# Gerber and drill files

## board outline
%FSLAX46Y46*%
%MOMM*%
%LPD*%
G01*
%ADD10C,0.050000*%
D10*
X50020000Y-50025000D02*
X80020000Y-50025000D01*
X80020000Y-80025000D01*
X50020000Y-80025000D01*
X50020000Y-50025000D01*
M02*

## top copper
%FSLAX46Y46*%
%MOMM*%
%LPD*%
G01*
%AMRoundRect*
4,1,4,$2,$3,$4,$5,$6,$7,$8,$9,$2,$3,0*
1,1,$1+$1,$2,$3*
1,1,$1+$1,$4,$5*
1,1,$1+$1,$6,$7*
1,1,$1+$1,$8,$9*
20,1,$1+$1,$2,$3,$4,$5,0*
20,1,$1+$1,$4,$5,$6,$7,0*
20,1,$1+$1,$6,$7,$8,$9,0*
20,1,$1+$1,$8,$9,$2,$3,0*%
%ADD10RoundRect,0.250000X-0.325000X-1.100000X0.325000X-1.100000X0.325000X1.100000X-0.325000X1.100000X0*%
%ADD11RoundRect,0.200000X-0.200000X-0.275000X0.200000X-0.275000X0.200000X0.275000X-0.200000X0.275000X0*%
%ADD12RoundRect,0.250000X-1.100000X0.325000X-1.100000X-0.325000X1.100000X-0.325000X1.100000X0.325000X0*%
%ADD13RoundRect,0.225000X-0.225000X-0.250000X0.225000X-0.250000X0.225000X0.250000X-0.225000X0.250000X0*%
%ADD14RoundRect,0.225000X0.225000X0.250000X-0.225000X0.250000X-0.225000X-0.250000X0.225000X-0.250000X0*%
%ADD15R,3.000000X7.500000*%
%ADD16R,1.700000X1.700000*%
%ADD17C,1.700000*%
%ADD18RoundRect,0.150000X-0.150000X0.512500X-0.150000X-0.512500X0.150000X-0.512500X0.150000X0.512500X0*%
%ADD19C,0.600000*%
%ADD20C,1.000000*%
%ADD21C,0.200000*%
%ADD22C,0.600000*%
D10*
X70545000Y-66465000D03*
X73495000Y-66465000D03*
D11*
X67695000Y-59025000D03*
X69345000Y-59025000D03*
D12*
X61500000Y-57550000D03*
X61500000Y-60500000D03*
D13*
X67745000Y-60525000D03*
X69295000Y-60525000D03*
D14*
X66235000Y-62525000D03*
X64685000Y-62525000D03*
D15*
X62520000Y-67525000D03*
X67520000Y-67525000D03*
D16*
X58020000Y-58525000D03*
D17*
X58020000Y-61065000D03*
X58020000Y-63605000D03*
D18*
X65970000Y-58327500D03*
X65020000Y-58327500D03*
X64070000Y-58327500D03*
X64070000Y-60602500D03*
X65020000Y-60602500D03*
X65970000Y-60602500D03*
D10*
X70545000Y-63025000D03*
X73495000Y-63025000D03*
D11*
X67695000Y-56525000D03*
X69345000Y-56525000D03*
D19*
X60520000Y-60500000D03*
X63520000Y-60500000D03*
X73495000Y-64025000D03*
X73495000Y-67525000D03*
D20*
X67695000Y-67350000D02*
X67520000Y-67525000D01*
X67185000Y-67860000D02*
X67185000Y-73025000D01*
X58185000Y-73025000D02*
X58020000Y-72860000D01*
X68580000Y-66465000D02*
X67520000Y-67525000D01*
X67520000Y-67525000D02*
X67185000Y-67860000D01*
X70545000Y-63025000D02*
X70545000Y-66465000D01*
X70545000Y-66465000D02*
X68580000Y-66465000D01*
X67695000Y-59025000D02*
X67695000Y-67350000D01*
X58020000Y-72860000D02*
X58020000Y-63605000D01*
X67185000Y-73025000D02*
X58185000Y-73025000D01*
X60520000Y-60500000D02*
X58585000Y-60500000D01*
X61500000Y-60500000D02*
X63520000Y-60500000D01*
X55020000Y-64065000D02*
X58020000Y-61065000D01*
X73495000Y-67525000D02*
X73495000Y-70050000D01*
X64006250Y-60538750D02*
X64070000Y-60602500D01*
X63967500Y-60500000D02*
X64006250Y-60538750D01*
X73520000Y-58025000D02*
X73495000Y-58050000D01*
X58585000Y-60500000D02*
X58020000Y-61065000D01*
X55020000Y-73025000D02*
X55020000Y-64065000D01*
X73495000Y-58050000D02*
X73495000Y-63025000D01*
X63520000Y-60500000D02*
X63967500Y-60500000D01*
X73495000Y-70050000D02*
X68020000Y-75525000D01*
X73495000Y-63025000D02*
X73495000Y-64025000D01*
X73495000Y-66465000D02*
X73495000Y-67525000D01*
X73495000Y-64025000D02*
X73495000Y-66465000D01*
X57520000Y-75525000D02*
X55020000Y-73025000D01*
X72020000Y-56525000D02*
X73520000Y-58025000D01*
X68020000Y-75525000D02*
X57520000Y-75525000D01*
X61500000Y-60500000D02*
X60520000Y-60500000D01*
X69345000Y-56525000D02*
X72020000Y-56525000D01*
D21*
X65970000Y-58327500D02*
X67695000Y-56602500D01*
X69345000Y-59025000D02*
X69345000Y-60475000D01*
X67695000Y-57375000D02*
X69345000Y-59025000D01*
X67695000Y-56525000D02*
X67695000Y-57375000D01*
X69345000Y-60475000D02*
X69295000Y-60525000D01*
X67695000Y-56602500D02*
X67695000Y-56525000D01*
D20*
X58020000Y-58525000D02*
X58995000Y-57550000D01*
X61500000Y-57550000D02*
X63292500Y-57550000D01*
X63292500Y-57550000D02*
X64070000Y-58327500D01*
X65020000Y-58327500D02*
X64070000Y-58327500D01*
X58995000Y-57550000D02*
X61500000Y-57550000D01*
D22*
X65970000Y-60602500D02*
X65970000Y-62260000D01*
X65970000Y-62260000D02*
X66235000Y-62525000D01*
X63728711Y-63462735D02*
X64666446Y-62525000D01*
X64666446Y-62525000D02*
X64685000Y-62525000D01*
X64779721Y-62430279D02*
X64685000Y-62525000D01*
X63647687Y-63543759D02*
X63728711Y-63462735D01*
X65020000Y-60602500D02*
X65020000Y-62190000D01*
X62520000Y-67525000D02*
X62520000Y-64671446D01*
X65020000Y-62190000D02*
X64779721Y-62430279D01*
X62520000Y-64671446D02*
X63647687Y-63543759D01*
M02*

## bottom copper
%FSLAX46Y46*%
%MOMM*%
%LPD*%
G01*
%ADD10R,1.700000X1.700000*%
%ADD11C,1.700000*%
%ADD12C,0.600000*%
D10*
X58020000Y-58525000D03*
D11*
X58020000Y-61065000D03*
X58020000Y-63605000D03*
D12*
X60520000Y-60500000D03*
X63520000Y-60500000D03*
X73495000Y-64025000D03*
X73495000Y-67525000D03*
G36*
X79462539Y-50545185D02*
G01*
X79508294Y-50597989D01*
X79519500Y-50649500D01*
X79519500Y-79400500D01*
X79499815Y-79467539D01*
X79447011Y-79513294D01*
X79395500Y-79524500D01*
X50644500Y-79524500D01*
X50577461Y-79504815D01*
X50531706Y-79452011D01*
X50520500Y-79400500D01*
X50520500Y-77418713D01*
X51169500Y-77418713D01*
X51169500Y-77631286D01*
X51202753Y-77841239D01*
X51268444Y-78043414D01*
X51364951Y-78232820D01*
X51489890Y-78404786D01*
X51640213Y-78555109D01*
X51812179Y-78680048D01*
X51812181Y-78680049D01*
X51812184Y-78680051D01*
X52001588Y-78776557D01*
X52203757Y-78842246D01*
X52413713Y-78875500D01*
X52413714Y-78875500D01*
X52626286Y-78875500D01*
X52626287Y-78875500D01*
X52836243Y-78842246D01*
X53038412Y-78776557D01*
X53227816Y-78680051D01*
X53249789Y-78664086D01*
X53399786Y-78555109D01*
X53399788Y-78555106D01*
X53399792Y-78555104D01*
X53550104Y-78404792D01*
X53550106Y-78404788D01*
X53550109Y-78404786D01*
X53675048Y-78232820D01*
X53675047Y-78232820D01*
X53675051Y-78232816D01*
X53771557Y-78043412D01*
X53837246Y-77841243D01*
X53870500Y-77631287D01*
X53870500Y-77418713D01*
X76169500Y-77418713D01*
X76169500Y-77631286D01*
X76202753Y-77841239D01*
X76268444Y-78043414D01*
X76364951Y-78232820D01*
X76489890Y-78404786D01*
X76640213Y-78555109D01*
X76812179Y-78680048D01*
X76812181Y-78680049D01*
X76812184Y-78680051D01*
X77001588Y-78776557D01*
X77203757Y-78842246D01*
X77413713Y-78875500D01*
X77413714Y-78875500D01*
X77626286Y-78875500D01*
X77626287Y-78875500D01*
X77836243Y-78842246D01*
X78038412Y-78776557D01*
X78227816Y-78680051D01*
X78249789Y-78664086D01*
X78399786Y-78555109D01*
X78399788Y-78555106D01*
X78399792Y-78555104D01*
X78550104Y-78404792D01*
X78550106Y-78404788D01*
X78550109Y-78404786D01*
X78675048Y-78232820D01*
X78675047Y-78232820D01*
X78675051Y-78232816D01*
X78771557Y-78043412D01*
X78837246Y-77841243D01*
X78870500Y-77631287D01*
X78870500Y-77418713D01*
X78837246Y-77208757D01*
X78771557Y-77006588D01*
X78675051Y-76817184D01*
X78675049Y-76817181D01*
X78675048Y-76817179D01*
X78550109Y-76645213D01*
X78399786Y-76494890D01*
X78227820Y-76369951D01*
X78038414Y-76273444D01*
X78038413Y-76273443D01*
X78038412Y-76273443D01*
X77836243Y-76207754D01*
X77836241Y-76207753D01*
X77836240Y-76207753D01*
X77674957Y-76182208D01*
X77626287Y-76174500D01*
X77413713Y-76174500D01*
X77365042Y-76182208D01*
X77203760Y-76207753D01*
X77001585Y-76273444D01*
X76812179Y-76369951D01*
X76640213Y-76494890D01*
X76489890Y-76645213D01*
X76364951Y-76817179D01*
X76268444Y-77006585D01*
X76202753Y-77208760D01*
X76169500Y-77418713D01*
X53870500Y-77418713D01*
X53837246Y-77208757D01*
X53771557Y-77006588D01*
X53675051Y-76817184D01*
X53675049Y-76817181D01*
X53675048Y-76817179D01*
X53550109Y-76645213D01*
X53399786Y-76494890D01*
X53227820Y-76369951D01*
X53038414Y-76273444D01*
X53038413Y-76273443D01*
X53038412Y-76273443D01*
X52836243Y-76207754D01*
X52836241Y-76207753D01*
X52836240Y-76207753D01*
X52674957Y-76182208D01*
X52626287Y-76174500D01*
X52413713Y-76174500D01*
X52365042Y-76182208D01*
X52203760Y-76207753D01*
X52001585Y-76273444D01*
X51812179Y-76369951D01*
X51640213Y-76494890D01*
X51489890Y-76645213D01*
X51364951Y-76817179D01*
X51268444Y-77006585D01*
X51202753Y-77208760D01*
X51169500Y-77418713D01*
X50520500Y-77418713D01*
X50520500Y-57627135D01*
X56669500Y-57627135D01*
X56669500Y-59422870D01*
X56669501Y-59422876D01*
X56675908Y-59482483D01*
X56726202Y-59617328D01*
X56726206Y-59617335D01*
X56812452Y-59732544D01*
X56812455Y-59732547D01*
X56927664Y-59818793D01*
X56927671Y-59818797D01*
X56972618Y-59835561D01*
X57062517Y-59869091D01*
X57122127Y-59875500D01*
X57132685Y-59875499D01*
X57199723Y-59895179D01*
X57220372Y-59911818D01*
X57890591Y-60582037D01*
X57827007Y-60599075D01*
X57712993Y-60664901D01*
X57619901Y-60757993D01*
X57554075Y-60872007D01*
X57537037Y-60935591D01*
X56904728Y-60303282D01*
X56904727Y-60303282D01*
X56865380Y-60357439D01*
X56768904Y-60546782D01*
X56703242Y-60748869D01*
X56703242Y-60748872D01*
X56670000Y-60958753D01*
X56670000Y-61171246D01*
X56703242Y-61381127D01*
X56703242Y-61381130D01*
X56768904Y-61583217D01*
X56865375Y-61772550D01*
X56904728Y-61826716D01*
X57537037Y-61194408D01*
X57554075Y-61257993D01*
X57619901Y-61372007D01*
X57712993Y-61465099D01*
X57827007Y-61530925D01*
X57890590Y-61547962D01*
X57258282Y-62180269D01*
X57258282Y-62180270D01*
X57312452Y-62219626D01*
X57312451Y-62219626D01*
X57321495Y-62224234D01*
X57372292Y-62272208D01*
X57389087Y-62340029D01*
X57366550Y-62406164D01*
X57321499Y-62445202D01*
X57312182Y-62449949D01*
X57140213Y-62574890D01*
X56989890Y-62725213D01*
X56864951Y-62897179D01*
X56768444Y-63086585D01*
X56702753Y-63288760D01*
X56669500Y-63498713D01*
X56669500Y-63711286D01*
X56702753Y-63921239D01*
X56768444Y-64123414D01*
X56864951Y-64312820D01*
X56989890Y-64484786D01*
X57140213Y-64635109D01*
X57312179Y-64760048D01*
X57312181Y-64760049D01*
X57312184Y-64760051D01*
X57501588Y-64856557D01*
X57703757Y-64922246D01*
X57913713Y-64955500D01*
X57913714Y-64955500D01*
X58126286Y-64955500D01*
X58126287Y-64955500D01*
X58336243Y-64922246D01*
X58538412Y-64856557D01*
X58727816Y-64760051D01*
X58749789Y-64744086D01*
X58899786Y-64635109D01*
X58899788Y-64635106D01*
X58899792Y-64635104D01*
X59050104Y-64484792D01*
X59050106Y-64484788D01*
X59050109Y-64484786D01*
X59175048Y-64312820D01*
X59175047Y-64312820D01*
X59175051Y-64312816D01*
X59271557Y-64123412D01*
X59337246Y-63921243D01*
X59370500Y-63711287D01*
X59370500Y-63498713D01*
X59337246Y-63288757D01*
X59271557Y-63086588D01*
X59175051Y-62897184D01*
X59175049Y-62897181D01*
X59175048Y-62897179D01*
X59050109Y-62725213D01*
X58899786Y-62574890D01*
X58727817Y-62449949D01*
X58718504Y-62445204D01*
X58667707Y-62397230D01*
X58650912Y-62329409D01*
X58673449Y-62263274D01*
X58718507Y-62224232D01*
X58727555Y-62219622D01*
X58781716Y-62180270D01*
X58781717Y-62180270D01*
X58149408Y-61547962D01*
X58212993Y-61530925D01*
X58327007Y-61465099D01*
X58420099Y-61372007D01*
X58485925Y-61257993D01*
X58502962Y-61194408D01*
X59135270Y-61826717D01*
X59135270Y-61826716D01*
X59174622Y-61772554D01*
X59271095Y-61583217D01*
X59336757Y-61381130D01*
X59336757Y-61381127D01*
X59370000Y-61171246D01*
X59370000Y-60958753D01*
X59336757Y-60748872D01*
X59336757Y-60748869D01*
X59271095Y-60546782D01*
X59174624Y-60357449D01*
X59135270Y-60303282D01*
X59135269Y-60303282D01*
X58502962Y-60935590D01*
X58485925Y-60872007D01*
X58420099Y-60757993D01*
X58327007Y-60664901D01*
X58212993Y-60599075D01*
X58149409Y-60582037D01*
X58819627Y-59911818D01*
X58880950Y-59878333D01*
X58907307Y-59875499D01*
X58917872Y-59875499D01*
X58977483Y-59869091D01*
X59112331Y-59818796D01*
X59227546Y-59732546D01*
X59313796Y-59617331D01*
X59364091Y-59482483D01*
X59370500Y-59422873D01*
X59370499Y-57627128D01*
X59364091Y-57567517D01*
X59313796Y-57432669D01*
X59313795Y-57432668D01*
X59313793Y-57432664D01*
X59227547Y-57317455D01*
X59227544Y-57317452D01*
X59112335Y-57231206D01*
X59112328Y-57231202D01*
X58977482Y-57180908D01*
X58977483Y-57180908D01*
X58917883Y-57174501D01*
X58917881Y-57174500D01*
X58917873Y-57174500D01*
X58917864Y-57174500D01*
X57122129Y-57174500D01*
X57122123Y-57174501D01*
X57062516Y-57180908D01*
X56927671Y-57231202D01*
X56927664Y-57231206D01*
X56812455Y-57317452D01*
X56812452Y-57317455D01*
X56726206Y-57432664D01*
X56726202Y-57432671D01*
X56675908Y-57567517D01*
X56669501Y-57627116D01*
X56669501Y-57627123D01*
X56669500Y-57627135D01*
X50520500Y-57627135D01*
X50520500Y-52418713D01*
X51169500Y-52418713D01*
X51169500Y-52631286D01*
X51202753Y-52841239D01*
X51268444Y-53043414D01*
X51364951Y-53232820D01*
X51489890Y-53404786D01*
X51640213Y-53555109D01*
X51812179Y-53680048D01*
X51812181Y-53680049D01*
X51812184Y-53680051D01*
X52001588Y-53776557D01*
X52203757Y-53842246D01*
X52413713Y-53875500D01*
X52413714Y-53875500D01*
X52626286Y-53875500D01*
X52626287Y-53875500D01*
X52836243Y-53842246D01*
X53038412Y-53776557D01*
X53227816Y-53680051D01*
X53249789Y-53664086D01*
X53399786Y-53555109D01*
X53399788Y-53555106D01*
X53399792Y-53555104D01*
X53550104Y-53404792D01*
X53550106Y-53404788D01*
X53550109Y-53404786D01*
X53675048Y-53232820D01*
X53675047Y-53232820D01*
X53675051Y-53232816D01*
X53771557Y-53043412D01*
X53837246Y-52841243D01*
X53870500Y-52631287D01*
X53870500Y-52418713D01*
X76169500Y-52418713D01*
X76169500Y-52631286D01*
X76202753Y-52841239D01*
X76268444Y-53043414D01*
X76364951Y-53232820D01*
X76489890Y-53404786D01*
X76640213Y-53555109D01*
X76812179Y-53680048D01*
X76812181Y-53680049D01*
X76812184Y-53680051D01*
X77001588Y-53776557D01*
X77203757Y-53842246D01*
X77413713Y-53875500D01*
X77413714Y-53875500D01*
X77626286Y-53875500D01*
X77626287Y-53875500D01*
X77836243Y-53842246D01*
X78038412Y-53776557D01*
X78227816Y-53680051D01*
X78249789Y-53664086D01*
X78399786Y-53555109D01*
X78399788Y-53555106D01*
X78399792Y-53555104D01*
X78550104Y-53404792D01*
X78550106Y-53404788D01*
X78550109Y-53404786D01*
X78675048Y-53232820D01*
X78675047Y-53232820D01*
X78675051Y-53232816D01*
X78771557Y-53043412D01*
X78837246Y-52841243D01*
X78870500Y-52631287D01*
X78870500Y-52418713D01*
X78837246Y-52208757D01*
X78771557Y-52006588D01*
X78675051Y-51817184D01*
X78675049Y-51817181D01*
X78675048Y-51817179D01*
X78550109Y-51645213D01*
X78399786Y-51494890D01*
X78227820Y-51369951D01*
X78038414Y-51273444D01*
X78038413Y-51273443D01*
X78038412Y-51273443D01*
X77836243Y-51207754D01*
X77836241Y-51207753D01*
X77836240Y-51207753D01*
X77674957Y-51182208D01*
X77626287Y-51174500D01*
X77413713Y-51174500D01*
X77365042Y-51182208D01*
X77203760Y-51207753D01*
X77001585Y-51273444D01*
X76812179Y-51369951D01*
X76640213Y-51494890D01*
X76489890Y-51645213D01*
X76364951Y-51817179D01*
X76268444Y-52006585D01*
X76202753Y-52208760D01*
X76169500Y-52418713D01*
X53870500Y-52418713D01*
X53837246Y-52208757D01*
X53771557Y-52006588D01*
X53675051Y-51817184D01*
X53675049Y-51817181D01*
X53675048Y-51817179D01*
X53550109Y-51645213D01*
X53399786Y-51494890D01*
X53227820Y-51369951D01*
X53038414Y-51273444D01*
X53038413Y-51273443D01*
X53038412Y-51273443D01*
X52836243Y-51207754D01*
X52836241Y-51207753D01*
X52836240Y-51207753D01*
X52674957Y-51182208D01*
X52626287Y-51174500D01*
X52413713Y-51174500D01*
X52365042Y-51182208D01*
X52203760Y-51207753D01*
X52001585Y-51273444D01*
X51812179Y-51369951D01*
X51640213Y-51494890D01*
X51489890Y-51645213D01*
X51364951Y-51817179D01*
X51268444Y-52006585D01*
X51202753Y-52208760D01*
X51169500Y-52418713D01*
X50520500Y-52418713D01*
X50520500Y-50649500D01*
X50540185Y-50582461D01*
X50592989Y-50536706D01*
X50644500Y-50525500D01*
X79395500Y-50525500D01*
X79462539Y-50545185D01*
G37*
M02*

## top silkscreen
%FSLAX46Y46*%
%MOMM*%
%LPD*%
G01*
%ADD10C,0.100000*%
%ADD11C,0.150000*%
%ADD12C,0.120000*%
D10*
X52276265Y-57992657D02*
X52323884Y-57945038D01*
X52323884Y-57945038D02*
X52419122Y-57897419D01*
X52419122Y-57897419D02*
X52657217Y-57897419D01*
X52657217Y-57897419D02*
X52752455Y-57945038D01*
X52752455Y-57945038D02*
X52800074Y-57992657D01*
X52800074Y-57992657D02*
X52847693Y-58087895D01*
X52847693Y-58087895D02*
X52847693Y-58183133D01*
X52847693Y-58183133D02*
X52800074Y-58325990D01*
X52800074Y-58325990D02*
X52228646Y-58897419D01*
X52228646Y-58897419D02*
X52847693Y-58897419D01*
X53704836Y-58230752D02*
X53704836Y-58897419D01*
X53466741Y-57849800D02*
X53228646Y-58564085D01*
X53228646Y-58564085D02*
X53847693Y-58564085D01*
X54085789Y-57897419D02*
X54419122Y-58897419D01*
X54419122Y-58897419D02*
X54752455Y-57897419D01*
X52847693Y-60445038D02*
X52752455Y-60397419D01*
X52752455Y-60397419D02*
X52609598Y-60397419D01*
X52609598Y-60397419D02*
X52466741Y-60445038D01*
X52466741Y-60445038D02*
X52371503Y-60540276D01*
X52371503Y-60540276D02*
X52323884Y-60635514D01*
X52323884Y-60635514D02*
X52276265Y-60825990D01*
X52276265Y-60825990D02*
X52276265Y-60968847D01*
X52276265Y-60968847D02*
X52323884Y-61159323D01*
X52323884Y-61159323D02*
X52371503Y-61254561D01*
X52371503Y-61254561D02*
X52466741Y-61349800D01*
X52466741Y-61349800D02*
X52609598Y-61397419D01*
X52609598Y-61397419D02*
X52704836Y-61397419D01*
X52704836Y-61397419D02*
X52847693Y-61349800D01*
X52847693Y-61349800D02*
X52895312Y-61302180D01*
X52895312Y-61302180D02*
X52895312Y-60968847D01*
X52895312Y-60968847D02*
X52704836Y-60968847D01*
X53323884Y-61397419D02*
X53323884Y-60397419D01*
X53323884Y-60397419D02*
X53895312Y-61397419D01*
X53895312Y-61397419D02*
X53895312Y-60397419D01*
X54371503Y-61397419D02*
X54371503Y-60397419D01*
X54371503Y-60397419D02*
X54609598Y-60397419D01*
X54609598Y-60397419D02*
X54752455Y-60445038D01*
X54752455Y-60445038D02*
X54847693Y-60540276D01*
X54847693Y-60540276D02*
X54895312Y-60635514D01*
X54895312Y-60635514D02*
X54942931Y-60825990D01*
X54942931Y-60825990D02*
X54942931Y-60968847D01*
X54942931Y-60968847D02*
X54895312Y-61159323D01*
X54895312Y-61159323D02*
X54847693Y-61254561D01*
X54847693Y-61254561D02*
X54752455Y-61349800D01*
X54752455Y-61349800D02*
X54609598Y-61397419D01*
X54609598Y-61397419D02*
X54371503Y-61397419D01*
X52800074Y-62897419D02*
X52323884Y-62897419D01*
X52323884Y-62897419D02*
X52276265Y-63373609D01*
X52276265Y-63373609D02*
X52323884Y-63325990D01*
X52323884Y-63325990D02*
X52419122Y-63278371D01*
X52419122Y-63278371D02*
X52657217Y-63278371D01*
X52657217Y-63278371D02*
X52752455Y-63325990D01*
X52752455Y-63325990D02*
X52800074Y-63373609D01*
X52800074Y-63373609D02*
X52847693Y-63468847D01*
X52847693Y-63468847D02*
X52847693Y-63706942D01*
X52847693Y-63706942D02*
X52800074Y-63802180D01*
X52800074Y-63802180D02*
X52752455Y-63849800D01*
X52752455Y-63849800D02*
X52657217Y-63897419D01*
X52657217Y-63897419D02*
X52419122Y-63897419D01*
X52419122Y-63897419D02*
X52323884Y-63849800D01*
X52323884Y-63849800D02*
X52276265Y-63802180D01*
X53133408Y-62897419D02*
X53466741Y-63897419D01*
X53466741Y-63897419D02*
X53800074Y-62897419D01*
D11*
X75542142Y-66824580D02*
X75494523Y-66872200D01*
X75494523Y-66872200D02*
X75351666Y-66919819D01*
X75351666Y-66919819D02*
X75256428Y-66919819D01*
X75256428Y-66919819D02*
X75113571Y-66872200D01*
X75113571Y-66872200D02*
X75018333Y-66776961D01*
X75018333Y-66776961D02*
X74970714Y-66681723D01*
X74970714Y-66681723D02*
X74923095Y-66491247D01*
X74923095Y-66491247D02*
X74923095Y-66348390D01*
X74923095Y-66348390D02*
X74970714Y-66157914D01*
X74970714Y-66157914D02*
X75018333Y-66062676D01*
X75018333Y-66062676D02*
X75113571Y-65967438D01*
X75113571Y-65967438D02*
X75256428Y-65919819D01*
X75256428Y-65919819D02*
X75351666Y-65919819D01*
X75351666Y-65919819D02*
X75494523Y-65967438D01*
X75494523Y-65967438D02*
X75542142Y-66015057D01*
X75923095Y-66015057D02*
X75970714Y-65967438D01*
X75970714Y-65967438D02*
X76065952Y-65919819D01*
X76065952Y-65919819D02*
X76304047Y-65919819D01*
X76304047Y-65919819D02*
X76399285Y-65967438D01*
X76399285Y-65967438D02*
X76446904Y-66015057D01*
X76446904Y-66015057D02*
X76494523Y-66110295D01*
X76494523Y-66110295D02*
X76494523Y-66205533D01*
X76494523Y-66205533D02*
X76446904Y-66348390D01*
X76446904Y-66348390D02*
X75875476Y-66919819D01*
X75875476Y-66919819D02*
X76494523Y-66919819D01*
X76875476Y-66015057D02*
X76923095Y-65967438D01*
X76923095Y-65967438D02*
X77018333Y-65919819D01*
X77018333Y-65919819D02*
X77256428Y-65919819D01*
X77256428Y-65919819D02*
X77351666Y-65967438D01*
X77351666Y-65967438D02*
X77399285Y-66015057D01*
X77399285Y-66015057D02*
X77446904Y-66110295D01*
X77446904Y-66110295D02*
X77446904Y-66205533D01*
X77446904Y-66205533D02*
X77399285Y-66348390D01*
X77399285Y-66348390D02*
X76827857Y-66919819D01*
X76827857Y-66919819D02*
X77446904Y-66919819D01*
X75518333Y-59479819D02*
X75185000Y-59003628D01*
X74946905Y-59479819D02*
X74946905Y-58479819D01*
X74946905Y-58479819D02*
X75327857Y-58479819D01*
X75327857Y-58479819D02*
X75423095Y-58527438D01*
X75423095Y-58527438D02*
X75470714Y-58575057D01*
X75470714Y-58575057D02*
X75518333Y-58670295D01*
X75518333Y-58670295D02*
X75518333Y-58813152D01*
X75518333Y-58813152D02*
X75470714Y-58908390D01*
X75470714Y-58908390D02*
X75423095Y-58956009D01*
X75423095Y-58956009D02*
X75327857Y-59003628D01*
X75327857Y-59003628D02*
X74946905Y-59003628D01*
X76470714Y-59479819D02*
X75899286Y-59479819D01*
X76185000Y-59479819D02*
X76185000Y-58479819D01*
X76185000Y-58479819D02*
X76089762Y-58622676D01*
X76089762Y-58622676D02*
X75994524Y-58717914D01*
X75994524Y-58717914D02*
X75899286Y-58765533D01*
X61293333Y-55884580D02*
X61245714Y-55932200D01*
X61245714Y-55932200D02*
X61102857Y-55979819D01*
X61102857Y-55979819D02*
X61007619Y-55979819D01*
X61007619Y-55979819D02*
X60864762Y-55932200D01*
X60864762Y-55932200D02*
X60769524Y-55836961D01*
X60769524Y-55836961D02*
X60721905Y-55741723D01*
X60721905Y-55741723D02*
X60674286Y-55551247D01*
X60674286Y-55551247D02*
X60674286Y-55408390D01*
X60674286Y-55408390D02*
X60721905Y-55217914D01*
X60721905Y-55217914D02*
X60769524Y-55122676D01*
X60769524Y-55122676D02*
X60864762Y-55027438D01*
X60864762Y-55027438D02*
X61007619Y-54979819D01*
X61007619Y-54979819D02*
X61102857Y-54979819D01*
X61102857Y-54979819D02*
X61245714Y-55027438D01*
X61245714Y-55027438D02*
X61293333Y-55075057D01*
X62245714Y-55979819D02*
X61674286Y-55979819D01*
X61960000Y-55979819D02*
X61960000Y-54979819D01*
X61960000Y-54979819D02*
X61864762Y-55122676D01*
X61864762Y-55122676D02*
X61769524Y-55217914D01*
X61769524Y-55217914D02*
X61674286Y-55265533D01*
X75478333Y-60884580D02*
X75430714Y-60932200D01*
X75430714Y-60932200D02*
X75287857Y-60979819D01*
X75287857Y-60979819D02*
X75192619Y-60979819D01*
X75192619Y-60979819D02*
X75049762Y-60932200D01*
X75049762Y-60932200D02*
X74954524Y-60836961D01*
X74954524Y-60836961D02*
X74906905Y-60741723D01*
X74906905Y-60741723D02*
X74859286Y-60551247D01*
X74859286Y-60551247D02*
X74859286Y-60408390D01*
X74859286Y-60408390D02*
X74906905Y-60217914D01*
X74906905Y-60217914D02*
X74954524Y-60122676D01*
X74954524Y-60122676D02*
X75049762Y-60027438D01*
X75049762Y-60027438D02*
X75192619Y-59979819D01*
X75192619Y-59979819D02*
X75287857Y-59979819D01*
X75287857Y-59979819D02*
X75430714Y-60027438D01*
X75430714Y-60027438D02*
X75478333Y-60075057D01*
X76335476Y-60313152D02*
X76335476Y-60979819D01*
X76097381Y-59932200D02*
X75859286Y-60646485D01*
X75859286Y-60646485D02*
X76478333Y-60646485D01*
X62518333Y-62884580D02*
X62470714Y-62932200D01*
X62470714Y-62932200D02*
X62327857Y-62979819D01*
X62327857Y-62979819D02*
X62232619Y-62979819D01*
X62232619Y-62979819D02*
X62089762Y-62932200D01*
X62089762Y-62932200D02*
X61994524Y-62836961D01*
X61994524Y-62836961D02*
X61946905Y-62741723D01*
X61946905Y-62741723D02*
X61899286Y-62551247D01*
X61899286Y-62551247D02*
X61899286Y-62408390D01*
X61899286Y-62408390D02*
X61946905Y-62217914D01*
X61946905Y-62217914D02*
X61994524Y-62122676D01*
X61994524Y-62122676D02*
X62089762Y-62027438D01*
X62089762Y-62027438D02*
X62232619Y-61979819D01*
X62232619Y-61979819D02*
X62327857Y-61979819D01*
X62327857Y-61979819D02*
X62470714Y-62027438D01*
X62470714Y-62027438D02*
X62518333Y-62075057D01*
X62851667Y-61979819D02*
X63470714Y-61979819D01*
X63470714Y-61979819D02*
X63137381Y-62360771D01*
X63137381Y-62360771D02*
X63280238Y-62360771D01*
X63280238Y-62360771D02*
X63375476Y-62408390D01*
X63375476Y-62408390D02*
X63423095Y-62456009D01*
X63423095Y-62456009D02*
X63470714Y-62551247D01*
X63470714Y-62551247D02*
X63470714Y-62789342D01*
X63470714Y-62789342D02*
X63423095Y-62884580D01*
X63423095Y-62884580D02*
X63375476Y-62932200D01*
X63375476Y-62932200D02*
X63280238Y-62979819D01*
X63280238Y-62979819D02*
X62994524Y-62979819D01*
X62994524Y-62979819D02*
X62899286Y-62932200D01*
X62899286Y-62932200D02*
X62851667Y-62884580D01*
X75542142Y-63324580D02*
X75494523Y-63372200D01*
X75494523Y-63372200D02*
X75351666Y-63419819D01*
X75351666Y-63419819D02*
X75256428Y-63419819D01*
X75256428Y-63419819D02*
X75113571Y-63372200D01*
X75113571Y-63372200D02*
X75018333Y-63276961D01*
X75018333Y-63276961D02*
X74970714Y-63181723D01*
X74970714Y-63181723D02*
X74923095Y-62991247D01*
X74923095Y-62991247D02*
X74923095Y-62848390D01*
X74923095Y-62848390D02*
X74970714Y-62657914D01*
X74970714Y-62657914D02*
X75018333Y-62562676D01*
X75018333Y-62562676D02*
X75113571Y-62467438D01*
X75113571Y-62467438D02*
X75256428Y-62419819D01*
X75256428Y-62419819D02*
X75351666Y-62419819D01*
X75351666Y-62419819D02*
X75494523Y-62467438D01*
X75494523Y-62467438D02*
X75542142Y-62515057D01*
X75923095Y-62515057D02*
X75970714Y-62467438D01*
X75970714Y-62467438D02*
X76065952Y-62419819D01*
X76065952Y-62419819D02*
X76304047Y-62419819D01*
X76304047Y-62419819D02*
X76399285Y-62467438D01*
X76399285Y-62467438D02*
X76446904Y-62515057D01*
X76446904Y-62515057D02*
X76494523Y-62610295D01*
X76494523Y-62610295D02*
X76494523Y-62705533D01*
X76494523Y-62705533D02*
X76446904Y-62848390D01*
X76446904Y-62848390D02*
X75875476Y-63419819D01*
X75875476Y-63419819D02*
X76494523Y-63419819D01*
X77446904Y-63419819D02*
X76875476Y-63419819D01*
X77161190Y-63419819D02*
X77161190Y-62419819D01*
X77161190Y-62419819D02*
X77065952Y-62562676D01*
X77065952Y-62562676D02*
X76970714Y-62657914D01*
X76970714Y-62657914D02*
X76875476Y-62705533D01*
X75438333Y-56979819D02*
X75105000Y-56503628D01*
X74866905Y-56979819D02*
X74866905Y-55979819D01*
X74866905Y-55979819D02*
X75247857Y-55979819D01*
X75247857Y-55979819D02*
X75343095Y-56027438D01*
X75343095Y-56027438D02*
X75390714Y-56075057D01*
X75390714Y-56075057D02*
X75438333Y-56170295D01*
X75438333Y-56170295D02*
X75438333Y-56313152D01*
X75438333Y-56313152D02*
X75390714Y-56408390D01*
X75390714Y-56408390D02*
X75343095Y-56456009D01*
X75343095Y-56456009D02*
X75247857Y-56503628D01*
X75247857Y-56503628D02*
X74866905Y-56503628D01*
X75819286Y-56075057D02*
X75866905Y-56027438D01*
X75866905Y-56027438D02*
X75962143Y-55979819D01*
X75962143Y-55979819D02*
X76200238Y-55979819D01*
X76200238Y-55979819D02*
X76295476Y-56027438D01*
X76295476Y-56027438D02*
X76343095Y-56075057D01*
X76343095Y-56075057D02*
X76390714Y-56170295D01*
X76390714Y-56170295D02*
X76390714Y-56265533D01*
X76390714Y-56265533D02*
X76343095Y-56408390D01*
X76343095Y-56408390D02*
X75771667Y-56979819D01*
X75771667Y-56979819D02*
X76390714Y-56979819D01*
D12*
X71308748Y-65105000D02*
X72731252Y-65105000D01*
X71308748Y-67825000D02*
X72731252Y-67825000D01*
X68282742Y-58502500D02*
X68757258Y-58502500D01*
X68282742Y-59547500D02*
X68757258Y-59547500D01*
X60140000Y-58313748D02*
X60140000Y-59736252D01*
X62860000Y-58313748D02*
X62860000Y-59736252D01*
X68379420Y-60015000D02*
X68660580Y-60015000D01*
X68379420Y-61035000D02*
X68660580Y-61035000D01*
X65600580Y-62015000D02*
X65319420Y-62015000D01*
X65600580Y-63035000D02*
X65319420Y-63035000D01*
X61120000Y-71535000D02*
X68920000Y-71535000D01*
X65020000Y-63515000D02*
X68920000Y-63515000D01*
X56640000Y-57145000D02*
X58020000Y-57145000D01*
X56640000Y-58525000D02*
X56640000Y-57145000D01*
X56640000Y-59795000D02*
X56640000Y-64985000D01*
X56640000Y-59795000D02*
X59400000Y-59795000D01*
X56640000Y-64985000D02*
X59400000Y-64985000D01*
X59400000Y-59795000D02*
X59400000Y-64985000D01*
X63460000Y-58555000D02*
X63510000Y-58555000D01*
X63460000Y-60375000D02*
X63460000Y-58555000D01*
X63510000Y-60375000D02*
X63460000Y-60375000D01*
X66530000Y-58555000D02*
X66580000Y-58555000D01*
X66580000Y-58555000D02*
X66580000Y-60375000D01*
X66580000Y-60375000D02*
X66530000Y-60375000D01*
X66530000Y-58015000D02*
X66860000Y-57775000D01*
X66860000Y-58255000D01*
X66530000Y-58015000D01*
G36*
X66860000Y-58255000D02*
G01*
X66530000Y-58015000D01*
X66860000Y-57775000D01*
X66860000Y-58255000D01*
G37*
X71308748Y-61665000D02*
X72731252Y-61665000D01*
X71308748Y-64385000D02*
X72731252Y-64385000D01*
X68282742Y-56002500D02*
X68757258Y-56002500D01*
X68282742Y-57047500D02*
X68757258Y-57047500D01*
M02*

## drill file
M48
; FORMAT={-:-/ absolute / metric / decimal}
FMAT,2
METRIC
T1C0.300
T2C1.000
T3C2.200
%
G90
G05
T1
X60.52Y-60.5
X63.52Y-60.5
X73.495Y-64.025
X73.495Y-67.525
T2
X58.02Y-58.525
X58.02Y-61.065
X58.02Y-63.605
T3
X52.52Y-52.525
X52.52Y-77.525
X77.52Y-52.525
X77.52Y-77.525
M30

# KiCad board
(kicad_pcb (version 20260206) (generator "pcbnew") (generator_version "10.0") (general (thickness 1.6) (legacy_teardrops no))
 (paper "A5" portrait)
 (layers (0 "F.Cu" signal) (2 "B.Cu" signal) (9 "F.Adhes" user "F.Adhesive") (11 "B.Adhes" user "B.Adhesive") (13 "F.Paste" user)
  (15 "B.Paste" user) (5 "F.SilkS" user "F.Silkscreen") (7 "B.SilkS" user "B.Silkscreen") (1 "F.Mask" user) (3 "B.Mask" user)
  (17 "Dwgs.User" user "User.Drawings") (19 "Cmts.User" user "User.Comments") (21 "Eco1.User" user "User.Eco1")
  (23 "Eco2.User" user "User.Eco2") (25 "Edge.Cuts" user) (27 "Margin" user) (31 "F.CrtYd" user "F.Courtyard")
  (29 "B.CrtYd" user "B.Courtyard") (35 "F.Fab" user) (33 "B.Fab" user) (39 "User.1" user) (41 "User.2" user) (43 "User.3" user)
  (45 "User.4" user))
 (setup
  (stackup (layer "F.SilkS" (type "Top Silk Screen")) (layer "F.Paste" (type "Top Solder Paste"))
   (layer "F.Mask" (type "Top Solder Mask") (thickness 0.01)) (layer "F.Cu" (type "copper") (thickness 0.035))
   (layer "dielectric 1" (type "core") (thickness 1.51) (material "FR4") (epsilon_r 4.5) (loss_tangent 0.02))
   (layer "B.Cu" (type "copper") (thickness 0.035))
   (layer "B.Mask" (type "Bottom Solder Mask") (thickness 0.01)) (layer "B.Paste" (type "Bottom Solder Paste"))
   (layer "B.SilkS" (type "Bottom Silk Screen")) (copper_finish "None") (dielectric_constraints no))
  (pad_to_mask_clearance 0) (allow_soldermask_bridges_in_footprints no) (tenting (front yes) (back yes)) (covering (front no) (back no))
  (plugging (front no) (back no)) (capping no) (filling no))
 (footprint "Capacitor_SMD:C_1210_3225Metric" (layer "F.Cu") (at 72.02 66.465)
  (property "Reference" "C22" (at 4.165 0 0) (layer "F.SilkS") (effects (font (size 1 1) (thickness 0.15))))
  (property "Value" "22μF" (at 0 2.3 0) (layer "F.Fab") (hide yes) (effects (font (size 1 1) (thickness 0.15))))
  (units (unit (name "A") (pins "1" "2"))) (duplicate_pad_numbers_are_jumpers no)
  (fp_line (start -0.711252 -1.36) (end 0.711252 -1.36) (stroke (width 0.12) (type solid)) (layer "F.SilkS"))
  (fp_line (start -0.711252 1.36) (end 0.711252 1.36) (stroke (width 0.12) (type solid)) (layer "F.SilkS"))
  (pad "1" smd roundrect (at -1.475 0) (size 1.15 2.7) (layers "F.Cu" "F.Mask" "F.Paste") (roundrect_rratio 0.217391) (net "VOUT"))
  (pad "2" smd roundrect (at 1.475 0) (size 1.15 2.7) (layers "F.Cu" "F.Mask" "F.Paste") (roundrect_rratio 0.217391) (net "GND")))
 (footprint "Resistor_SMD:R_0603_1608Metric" (layer "F.Cu") (at 68.52 59.025)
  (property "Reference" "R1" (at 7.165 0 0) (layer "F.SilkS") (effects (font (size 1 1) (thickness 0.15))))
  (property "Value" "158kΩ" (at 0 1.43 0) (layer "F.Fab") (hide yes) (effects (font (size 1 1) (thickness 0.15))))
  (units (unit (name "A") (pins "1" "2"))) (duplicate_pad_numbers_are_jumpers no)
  (fp_line (start -0.237258 -0.5225) (end 0.237258 -0.5225) (stroke (width 0.12) (type solid)) (layer "F.SilkS"))
  (fp_line (start -0.237258 0.5225) (end 0.237258 0.5225) (stroke (width 0.12) (type solid)) (layer "F.SilkS"))
  (pad "1" smd roundrect (at -0.825 0) (size 0.8 0.95) (layers "F.Cu" "F.Mask" "F.Paste") (roundrect_rratio 0.25) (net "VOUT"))
  (pad "2" smd roundrect (at 0.825 0) (size 0.8 0.95) (layers "F.Cu" "F.Mask" "F.Paste") (roundrect_rratio 0.25) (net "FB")))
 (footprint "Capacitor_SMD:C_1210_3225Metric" (layer "F.Cu") (at 61.5 59.025 -90)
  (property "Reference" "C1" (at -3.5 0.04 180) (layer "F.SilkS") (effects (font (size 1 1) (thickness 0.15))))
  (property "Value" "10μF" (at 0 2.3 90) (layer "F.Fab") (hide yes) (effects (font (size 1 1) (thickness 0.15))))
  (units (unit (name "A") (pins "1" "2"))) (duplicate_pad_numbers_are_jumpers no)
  (fp_line (start -0.711252 1.36) (end 0.711252 1.36) (stroke (width 0.12) (type solid)) (layer "F.SilkS"))
  (fp_line (start -0.711252 -1.36) (end 0.711252 -1.36) (stroke (width 0.12) (type solid)) (layer "F.SilkS"))
  (pad "1" smd roundrect (at -1.475 0 270) (size 1.15 2.7) (layers "F.Cu" "F.Mask" "F.Paste") (roundrect_rratio 0.217391) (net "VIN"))
  (pad "2" smd roundrect (at 1.475 0 270) (size 1.15 2.7) (layers "F.Cu" "F.Mask" "F.Paste") (roundrect_rratio 0.217391) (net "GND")))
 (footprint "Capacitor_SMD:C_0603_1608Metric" (layer "F.Cu") (at 68.52 60.525)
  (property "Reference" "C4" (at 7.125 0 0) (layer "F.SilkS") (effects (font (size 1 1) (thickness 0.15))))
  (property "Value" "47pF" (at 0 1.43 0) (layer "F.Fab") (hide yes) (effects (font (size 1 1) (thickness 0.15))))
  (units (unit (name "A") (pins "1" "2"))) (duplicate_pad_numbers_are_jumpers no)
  (fp_line (start -0.14058 -0.51) (end 0.14058 -0.51) (stroke (width 0.12) (type solid)) (layer "F.SilkS"))
  (fp_line (start -0.14058 0.51) (end 0.14058 0.51) (stroke (width 0.12) (type solid)) (layer "F.SilkS"))
  (pad "1" smd roundrect (at -0.775 0) (size 0.9 0.95) (layers "F.Cu" "F.Mask" "F.Paste") (roundrect_rratio 0.25) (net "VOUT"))
  (pad "2" smd roundrect (at 0.775 0) (size 0.9 0.95) (layers "F.Cu" "F.Mask" "F.Paste") (roundrect_rratio 0.25) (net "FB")))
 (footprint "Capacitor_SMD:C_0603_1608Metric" (layer "F.Cu") (at 65.46 62.525 180)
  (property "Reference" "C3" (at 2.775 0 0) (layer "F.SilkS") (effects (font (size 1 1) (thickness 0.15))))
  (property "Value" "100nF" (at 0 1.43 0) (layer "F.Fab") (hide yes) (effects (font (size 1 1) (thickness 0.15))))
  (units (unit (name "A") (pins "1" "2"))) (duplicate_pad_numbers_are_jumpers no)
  (fp_line (start -0.14058 0.51) (end 0.14058 0.51) (stroke (width 0.12) (type solid)) (layer "F.SilkS"))
  (fp_line (start -0.14058 -0.51) (end 0.14058 -0.51) (stroke (width 0.12) (type solid)) (layer "F.SilkS"))
  (pad "1" smd roundrect (at -0.775 0 180) (size 0.9 0.95) (layers "F.Cu" "F.Mask" "F.Paste") (roundrect_rratio 0.25) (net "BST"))
  (pad "2" smd roundrect (at 0.775 0 180) (size 0.9 0.95) (layers "F.Cu" "F.Mask" "F.Paste") (roundrect_rratio 0.25) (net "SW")))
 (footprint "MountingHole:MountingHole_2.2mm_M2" (layer "F.Cu") (at 52.52 77.525)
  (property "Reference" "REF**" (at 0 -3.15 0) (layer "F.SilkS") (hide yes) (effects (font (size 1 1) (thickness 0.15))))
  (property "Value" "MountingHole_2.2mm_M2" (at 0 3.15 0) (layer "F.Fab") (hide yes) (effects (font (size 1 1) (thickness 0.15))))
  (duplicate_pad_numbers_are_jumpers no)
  (pad "" np_thru_hole circle (at 0 0) (size 2.2 2.2) (drill 2.2) (layers "*.Cu" "*.Mask")))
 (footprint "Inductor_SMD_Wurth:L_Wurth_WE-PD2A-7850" (layer "F.Cu") (at 65.02 67.525)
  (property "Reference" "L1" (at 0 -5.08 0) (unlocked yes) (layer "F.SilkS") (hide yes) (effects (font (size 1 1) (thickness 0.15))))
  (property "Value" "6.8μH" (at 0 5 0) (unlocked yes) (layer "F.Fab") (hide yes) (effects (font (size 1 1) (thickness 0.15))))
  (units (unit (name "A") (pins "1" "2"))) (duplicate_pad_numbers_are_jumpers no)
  (fp_line (start -3.9 4.01) (end 3.9 4.01) (stroke (width 0.12) (type solid)) (layer "F.SilkS"))
  (fp_line (start 0 -4.01) (end 3.9 -4.01) (stroke (width 0.12) (type solid)) (layer "F.SilkS"))
  (pad "1" smd rect (at -2.5 0) (size 3 7.5) (layers "F.Cu" "F.Mask" "F.Paste") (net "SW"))
  (pad "2" smd rect (at 2.5 0) (size 3 7.5) (layers "F.Cu" "F.Mask" "F.Paste") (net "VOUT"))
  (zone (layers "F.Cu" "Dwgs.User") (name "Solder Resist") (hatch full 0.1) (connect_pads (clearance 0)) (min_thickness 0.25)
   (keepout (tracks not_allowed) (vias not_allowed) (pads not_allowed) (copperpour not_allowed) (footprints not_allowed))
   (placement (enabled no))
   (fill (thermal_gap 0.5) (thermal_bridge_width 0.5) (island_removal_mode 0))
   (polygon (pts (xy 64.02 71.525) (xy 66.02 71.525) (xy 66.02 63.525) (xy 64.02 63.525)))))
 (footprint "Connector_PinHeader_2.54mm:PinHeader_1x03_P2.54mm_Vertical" (layer "F.Cu") (at 58.02 58.525)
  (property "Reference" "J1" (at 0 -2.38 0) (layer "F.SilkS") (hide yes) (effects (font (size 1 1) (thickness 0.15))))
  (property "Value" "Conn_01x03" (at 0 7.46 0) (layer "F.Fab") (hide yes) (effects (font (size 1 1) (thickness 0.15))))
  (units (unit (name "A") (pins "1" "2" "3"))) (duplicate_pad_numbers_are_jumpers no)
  (fp_line (start -1.38 -1.38) (end 0 -1.38) (stroke (width 0.12) (type solid)) (layer "F.SilkS"))
  (fp_line (start -1.38 0) (end -1.38 -1.38) (stroke (width 0.12) (type solid)) (layer "F.SilkS"))
  (fp_line (start -1.38 1.27) (end -1.38 6.46) (stroke (width 0.12) (type solid)) (layer "F.SilkS"))
  (fp_line (start -1.38 1.27) (end 1.38 1.27) (stroke (width 0.12) (type solid)) (layer "F.SilkS"))
  (fp_line (start -1.38 6.46) (end 1.38 6.46) (stroke (width 0.12) (type solid)) (layer "F.SilkS"))
  (fp_line (start 1.38 1.27) (end 1.38 6.46) (stroke (width 0.12) (type solid)) (layer "F.SilkS"))
  (pad "1" thru_hole rect (at 0 0) (size 1.7 1.7) (drill 1) (layers "*.Cu" "*.Mask") (remove_unused_layers no) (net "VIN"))
  (pad "2" thru_hole circle (at 0 2.54) (size 1.7 1.7) (drill 1) (layers "*.Cu" "*.Mask") (remove_unused_layers no) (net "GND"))
  (pad "3" thru_hole circle (at 0 5.08) (size 1.7 1.7) (drill 1) (layers "*.Cu" "*.Mask") (remove_unused_layers no) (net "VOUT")))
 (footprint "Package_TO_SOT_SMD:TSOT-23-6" (layer "F.Cu") (at 65.02 59.465 -90)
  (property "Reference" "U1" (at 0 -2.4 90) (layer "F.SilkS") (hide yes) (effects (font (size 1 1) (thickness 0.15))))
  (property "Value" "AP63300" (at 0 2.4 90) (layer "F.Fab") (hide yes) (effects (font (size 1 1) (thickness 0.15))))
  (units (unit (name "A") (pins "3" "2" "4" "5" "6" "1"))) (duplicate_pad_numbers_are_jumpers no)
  (fp_line (start -0.91 1.56) (end -0.91 1.51) (stroke (width 0.12) (type solid)) (layer "F.SilkS"))
  (fp_line (start 0.91 1.56) (end -0.91 1.56) (stroke (width 0.12) (type solid)) (layer "F.SilkS"))
  (fp_line (start 0.91 1.51) (end 0.91 1.56) (stroke (width 0.12) (type solid)) (layer "F.SilkS"))
  (fp_line (start -0.91 -1.51) (end -0.91 -1.56) (stroke (width 0.12) (type solid)) (layer "F.SilkS"))
  (fp_line (start -0.91 -1.56) (end 0.91 -1.56) (stroke (width 0.12) (type solid)) (layer "F.SilkS"))
  (fp_line (start 0.91 -1.56) (end 0.91 -1.51) (stroke (width 0.12) (type solid)) (layer "F.SilkS"))
  (fp_poly (pts (xy -1.45 -1.51) (xy -1.69 -1.84) (xy -1.21 -1.84)) (stroke (width 0.12) (type solid)) (fill yes) (layer "F.SilkS"))
  (pad "1" smd roundrect (at -1.1375 -0.95 270) (size 1.325 0.6) (layers "F.Cu" "F.Mask" "F.Paste") (roundrect_rratio 0.25) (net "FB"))
  (pad "2" smd roundrect (at -1.1375 0 270) (size 1.325 0.6) (layers "F.Cu" "F.Mask" "F.Paste") (roundrect_rratio 0.25) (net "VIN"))
  (pad "3" smd roundrect (at -1.1375 0.95 270) (size 1.325 0.6) (layers "F.Cu" "F.Mask" "F.Paste") (roundrect_rratio 0.25) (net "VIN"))
  (pad "4" smd roundrect (at 1.1375 0.95 270) (size 1.325 0.6) (layers "F.Cu" "F.Mask" "F.Paste") (roundrect_rratio 0.25) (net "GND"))
  (pad "5" smd roundrect (at 1.1375 0 270) (size 1.325 0.6) (layers "F.Cu" "F.Mask" "F.Paste") (roundrect_rratio 0.25) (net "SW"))
  (pad "6" smd roundrect (at 1.1375 -0.95 270) (size 1.325 0.6) (layers "F.Cu" "F.Mask" "F.Paste") (roundrect_rratio 0.25) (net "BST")))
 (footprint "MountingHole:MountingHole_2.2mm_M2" (layer "F.Cu") (at 52.52 52.525)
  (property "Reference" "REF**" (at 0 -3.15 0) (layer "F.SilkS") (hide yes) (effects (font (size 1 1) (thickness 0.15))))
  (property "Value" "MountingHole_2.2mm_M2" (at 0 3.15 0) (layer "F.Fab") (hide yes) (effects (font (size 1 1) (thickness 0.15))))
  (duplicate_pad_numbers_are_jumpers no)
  (pad "" np_thru_hole circle (at 0 0) (size 2.2 2.2) (drill 2.2) (layers "*.Cu" "*.Mask")))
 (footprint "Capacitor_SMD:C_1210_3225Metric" (layer "F.Cu") (at 72.02 63.025)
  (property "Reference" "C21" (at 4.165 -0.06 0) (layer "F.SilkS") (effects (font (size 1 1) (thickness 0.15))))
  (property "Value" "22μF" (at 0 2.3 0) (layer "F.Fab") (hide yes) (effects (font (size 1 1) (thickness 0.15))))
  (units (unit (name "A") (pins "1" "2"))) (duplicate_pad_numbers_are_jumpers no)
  (fp_line (start -0.711252 -1.36) (end 0.711252 -1.36) (stroke (width 0.12) (type solid)) (layer "F.SilkS"))
  (fp_line (start -0.711252 1.36) (end 0.711252 1.36) (stroke (width 0.12) (type solid)) (layer "F.SilkS"))
  (pad "1" smd roundrect (at -1.475 0) (size 1.15 2.7) (layers "F.Cu" "F.Mask" "F.Paste") (roundrect_rratio 0.217391) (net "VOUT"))
  (pad "2" smd roundrect (at 1.475 0) (size 1.15 2.7) (layers "F.Cu" "F.Mask" "F.Paste") (roundrect_rratio 0.217391) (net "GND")))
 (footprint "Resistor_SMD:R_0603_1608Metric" (layer "F.Cu") (at 68.52 56.525)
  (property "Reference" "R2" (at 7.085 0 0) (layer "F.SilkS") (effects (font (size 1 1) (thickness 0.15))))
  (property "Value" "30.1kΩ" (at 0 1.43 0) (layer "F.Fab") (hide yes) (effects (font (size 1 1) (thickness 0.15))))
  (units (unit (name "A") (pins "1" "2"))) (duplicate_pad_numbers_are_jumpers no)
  (fp_line (start -0.237258 -0.5225) (end 0.237258 -0.5225) (stroke (width 0.12) (type solid)) (layer "F.SilkS"))
  (fp_line (start -0.237258 0.5225) (end 0.237258 0.5225) (stroke (width 0.12) (type solid)) (layer "F.SilkS"))
  (pad "1" smd roundrect (at -0.825 0) (size 0.8 0.95) (layers "F.Cu" "F.Mask" "F.Paste") (roundrect_rratio 0.25) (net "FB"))
  (pad "2" smd roundrect (at 0.825 0) (size 0.8 0.95) (layers "F.Cu" "F.Mask" "F.Paste") (roundrect_rratio 0.25) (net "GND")))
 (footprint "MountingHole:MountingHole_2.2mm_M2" (layer "F.Cu") (at 77.52 77.525)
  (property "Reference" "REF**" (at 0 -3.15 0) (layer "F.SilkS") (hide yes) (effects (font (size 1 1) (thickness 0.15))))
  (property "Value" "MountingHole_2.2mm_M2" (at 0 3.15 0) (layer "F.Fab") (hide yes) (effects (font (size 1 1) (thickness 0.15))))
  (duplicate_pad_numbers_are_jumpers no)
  (pad "" np_thru_hole circle (at 0 0) (size 2.2 2.2) (drill 2.2) (layers "*.Cu" "*.Mask")))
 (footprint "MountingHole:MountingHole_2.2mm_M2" (layer "F.Cu") (at 77.52 52.525)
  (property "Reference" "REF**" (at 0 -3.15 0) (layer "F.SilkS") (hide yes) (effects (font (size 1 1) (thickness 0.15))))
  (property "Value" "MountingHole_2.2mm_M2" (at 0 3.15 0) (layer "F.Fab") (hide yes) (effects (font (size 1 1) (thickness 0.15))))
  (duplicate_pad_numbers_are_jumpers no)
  (pad "" np_thru_hole circle (at 0 0) (size 2.2 2.2) (drill 2.2) (layers "*.Cu" "*.Mask")))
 (gr_rect (start 50.02 50.025) (end 80.02 80.025) (stroke (width 0.05) (type default)) (fill no) (layer "Edge.Cuts"))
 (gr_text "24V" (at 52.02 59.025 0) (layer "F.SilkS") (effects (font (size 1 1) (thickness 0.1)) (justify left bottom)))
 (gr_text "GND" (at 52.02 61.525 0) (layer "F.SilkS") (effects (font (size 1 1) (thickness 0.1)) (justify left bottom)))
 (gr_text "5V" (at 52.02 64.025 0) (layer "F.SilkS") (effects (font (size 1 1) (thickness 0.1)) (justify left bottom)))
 (segment (start 67.695 67.35) (end 67.52 67.525) (width 1) (layer "F.Cu") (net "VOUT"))
 (segment (start 67.185 67.86) (end 67.185 73.025) (width 1) (layer "F.Cu") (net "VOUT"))
 (segment (start 58.185 73.025) (end 58.02 72.86) (width 1) (layer "F.Cu") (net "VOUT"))
 (segment (start 68.58 66.465) (end 67.52 67.525) (width 1) (layer "F.Cu") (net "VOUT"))
 (segment (start 67.52 67.525) (end 67.185 67.86) (width 1) (layer "F.Cu") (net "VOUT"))
 (segment (start 70.545 63.025) (end 70.545 66.465) (width 1) (layer "F.Cu") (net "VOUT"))
 (segment (start 70.545 66.465) (end 68.58 66.465) (width 1) (layer "F.Cu") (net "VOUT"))
 (segment (start 67.695 59.025) (end 67.695 67.35) (width 1) (layer "F.Cu") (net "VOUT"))
 (segment (start 58.02 72.86) (end 58.02 63.605) (width 1) (layer "F.Cu") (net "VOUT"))
 (segment (start 67.185 73.025) (end 58.185 73.025) (width 1) (layer "F.Cu") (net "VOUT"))
 (segment (start 60.52 60.5) (end 58.585 60.5) (width 1) (layer "F.Cu") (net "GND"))
 (segment (start 61.5 60.5) (end 63.52 60.5) (width 1) (layer "F.Cu") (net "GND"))
 (segment (start 55.02 64.065) (end 58.02 61.065) (width 1) (layer "F.Cu") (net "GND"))
 (segment (start 73.495 67.525) (end 73.495 70.05) (width 1) (layer "F.Cu") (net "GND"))
 (segment (start 64.00625 60.53875) (end 64.07 60.6025) (width 1) (layer "F.Cu") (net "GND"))
 (segment (start 63.9675 60.5) (end 64.00625 60.53875) (width 1) (layer "F.Cu") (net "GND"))
 (segment (start 73.52 58.025) (end 73.495 58.05) (width 1) (layer "F.Cu") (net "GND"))
 (segment (start 58.585 60.5) (end 58.02 61.065) (width 1) (layer "F.Cu") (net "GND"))
 (segment (start 55.02 73.025) (end 55.02 64.065) (width 1) (layer "F.Cu") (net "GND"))
 (segment (start 73.495 58.05) (end 73.495 63.025) (width 1) (layer "F.Cu") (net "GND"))
 (segment (start 63.52 60.5) (end 63.9675 60.5) (width 1) (layer "F.Cu") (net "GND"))
 (segment (start 73.495 70.05) (end 68.02 75.525) (width 1) (layer "F.Cu") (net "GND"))
 (segment (start 73.495 63.025) (end 73.495 64.025) (width 1) (layer "F.Cu") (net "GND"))
 (segment (start 73.495 66.465) (end 73.495 67.525) (width 1) (layer "F.Cu") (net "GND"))
 (segment (start 73.495 64.025) (end 73.495 66.465) (width 1) (layer "F.Cu") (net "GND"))
 (segment (start 57.52 75.525) (end 55.02 73.025) (width 1) (layer "F.Cu") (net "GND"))
 (segment (start 72.02 56.525) (end 73.52 58.025) (width 1) (layer "F.Cu") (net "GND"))
 (segment (start 68.02 75.525) (end 57.52 75.525) (width 1) (layer "F.Cu") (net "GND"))
 (segment (start 61.5 60.5) (end 60.52 60.5) (width 1) (layer "F.Cu") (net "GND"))
 (segment (start 69.345 56.525) (end 72.02 56.525) (width 1) (layer "F.Cu") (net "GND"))
 (via (at 60.52 60.5) (size 0.6) (drill 0.3) (layers "F.Cu" "B.Cu") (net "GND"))
 (via (at 63.52 60.5) (size 0.6) (drill 0.3) (layers "F.Cu" "B.Cu") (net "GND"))
 (via (at 73.495 64.025) (size 0.6) (drill 0.3) (layers "F.Cu" "B.Cu") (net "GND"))
 (via (at 73.495 67.525) (size 0.6) (drill 0.3) (layers "F.Cu" "B.Cu") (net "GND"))
 (segment (start 65.97 58.3275) (end 67.695 56.6025) (width 0.2) (layer "F.Cu") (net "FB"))
 (segment (start 69.345 59.025) (end 69.345 60.475) (width 0.2) (layer "F.Cu") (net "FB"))
 (segment (start 67.695 57.375) (end 69.345 59.025) (width 0.2) (layer "F.Cu") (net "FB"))
 (segment (start 67.695 56.525) (end 67.695 57.375) (width 0.2) (layer "F.Cu") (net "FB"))
 (segment (start 69.345 60.475) (end 69.295 60.525) (width 0.2) (layer "F.Cu") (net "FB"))
 (segment (start 67.695 56.6025) (end 67.695 56.525) (width 0.2) (layer "F.Cu") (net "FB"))
 (segment (start 58.02 58.525) (end 58.995 57.55) (width 1) (layer "F.Cu") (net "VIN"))
 (segment (start 61.5 57.55) (end 63.2925 57.55) (width 1) (layer "F.Cu") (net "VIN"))
 (segment (start 63.2925 57.55) (end 64.07 58.3275) (width 1) (layer "F.Cu") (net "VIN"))
 (segment (start 65.02 58.3275) (end 64.07 58.3275) (width 1) (layer "F.Cu") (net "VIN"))
 (segment (start 58.995 57.55) (end 61.5 57.55) (width 1) (layer "F.Cu") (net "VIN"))
 (segment (start 65.97 60.6025) (end 65.97 62.26) (width 0.6) (layer "F.Cu") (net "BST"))
 (segment (start 65.97 62.26) (end 66.235 62.525) (width 0.6) (layer "F.Cu") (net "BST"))
 (segment (start 63.728711 63.462735) (end 64.666446 62.525) (width 0.6) (layer "F.Cu") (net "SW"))
 (segment (start 64.666446 62.525) (end 64.685 62.525) (width 0.6) (layer "F.Cu") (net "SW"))
 (segment (start 64.779721 62.430279) (end 64.685 62.525) (width 0.6) (layer "F.Cu") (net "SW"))
 (segment (start 63.647687 63.543759) (end 63.728711 63.462735) (width 0.6) (layer "F.Cu") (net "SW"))
 (segment (start 65.02 60.6025) (end 65.02 62.19) (width 0.6) (layer "F.Cu") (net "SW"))
 (segment (start 62.52 67.525) (end 62.52 64.671446) (width 0.6) (layer "F.Cu") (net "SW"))
 (segment (start 65.02 62.19) (end 64.779721 62.430279) (width 0.6) (layer "F.Cu") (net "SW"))
 (segment (start 62.52 64.671446) (end 63.647687 63.543759) (width 0.6) (layer "F.Cu") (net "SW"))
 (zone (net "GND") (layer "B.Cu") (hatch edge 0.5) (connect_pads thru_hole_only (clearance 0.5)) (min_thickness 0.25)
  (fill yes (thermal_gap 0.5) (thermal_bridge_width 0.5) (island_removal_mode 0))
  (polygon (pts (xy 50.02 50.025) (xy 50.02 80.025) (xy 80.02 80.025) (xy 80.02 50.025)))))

